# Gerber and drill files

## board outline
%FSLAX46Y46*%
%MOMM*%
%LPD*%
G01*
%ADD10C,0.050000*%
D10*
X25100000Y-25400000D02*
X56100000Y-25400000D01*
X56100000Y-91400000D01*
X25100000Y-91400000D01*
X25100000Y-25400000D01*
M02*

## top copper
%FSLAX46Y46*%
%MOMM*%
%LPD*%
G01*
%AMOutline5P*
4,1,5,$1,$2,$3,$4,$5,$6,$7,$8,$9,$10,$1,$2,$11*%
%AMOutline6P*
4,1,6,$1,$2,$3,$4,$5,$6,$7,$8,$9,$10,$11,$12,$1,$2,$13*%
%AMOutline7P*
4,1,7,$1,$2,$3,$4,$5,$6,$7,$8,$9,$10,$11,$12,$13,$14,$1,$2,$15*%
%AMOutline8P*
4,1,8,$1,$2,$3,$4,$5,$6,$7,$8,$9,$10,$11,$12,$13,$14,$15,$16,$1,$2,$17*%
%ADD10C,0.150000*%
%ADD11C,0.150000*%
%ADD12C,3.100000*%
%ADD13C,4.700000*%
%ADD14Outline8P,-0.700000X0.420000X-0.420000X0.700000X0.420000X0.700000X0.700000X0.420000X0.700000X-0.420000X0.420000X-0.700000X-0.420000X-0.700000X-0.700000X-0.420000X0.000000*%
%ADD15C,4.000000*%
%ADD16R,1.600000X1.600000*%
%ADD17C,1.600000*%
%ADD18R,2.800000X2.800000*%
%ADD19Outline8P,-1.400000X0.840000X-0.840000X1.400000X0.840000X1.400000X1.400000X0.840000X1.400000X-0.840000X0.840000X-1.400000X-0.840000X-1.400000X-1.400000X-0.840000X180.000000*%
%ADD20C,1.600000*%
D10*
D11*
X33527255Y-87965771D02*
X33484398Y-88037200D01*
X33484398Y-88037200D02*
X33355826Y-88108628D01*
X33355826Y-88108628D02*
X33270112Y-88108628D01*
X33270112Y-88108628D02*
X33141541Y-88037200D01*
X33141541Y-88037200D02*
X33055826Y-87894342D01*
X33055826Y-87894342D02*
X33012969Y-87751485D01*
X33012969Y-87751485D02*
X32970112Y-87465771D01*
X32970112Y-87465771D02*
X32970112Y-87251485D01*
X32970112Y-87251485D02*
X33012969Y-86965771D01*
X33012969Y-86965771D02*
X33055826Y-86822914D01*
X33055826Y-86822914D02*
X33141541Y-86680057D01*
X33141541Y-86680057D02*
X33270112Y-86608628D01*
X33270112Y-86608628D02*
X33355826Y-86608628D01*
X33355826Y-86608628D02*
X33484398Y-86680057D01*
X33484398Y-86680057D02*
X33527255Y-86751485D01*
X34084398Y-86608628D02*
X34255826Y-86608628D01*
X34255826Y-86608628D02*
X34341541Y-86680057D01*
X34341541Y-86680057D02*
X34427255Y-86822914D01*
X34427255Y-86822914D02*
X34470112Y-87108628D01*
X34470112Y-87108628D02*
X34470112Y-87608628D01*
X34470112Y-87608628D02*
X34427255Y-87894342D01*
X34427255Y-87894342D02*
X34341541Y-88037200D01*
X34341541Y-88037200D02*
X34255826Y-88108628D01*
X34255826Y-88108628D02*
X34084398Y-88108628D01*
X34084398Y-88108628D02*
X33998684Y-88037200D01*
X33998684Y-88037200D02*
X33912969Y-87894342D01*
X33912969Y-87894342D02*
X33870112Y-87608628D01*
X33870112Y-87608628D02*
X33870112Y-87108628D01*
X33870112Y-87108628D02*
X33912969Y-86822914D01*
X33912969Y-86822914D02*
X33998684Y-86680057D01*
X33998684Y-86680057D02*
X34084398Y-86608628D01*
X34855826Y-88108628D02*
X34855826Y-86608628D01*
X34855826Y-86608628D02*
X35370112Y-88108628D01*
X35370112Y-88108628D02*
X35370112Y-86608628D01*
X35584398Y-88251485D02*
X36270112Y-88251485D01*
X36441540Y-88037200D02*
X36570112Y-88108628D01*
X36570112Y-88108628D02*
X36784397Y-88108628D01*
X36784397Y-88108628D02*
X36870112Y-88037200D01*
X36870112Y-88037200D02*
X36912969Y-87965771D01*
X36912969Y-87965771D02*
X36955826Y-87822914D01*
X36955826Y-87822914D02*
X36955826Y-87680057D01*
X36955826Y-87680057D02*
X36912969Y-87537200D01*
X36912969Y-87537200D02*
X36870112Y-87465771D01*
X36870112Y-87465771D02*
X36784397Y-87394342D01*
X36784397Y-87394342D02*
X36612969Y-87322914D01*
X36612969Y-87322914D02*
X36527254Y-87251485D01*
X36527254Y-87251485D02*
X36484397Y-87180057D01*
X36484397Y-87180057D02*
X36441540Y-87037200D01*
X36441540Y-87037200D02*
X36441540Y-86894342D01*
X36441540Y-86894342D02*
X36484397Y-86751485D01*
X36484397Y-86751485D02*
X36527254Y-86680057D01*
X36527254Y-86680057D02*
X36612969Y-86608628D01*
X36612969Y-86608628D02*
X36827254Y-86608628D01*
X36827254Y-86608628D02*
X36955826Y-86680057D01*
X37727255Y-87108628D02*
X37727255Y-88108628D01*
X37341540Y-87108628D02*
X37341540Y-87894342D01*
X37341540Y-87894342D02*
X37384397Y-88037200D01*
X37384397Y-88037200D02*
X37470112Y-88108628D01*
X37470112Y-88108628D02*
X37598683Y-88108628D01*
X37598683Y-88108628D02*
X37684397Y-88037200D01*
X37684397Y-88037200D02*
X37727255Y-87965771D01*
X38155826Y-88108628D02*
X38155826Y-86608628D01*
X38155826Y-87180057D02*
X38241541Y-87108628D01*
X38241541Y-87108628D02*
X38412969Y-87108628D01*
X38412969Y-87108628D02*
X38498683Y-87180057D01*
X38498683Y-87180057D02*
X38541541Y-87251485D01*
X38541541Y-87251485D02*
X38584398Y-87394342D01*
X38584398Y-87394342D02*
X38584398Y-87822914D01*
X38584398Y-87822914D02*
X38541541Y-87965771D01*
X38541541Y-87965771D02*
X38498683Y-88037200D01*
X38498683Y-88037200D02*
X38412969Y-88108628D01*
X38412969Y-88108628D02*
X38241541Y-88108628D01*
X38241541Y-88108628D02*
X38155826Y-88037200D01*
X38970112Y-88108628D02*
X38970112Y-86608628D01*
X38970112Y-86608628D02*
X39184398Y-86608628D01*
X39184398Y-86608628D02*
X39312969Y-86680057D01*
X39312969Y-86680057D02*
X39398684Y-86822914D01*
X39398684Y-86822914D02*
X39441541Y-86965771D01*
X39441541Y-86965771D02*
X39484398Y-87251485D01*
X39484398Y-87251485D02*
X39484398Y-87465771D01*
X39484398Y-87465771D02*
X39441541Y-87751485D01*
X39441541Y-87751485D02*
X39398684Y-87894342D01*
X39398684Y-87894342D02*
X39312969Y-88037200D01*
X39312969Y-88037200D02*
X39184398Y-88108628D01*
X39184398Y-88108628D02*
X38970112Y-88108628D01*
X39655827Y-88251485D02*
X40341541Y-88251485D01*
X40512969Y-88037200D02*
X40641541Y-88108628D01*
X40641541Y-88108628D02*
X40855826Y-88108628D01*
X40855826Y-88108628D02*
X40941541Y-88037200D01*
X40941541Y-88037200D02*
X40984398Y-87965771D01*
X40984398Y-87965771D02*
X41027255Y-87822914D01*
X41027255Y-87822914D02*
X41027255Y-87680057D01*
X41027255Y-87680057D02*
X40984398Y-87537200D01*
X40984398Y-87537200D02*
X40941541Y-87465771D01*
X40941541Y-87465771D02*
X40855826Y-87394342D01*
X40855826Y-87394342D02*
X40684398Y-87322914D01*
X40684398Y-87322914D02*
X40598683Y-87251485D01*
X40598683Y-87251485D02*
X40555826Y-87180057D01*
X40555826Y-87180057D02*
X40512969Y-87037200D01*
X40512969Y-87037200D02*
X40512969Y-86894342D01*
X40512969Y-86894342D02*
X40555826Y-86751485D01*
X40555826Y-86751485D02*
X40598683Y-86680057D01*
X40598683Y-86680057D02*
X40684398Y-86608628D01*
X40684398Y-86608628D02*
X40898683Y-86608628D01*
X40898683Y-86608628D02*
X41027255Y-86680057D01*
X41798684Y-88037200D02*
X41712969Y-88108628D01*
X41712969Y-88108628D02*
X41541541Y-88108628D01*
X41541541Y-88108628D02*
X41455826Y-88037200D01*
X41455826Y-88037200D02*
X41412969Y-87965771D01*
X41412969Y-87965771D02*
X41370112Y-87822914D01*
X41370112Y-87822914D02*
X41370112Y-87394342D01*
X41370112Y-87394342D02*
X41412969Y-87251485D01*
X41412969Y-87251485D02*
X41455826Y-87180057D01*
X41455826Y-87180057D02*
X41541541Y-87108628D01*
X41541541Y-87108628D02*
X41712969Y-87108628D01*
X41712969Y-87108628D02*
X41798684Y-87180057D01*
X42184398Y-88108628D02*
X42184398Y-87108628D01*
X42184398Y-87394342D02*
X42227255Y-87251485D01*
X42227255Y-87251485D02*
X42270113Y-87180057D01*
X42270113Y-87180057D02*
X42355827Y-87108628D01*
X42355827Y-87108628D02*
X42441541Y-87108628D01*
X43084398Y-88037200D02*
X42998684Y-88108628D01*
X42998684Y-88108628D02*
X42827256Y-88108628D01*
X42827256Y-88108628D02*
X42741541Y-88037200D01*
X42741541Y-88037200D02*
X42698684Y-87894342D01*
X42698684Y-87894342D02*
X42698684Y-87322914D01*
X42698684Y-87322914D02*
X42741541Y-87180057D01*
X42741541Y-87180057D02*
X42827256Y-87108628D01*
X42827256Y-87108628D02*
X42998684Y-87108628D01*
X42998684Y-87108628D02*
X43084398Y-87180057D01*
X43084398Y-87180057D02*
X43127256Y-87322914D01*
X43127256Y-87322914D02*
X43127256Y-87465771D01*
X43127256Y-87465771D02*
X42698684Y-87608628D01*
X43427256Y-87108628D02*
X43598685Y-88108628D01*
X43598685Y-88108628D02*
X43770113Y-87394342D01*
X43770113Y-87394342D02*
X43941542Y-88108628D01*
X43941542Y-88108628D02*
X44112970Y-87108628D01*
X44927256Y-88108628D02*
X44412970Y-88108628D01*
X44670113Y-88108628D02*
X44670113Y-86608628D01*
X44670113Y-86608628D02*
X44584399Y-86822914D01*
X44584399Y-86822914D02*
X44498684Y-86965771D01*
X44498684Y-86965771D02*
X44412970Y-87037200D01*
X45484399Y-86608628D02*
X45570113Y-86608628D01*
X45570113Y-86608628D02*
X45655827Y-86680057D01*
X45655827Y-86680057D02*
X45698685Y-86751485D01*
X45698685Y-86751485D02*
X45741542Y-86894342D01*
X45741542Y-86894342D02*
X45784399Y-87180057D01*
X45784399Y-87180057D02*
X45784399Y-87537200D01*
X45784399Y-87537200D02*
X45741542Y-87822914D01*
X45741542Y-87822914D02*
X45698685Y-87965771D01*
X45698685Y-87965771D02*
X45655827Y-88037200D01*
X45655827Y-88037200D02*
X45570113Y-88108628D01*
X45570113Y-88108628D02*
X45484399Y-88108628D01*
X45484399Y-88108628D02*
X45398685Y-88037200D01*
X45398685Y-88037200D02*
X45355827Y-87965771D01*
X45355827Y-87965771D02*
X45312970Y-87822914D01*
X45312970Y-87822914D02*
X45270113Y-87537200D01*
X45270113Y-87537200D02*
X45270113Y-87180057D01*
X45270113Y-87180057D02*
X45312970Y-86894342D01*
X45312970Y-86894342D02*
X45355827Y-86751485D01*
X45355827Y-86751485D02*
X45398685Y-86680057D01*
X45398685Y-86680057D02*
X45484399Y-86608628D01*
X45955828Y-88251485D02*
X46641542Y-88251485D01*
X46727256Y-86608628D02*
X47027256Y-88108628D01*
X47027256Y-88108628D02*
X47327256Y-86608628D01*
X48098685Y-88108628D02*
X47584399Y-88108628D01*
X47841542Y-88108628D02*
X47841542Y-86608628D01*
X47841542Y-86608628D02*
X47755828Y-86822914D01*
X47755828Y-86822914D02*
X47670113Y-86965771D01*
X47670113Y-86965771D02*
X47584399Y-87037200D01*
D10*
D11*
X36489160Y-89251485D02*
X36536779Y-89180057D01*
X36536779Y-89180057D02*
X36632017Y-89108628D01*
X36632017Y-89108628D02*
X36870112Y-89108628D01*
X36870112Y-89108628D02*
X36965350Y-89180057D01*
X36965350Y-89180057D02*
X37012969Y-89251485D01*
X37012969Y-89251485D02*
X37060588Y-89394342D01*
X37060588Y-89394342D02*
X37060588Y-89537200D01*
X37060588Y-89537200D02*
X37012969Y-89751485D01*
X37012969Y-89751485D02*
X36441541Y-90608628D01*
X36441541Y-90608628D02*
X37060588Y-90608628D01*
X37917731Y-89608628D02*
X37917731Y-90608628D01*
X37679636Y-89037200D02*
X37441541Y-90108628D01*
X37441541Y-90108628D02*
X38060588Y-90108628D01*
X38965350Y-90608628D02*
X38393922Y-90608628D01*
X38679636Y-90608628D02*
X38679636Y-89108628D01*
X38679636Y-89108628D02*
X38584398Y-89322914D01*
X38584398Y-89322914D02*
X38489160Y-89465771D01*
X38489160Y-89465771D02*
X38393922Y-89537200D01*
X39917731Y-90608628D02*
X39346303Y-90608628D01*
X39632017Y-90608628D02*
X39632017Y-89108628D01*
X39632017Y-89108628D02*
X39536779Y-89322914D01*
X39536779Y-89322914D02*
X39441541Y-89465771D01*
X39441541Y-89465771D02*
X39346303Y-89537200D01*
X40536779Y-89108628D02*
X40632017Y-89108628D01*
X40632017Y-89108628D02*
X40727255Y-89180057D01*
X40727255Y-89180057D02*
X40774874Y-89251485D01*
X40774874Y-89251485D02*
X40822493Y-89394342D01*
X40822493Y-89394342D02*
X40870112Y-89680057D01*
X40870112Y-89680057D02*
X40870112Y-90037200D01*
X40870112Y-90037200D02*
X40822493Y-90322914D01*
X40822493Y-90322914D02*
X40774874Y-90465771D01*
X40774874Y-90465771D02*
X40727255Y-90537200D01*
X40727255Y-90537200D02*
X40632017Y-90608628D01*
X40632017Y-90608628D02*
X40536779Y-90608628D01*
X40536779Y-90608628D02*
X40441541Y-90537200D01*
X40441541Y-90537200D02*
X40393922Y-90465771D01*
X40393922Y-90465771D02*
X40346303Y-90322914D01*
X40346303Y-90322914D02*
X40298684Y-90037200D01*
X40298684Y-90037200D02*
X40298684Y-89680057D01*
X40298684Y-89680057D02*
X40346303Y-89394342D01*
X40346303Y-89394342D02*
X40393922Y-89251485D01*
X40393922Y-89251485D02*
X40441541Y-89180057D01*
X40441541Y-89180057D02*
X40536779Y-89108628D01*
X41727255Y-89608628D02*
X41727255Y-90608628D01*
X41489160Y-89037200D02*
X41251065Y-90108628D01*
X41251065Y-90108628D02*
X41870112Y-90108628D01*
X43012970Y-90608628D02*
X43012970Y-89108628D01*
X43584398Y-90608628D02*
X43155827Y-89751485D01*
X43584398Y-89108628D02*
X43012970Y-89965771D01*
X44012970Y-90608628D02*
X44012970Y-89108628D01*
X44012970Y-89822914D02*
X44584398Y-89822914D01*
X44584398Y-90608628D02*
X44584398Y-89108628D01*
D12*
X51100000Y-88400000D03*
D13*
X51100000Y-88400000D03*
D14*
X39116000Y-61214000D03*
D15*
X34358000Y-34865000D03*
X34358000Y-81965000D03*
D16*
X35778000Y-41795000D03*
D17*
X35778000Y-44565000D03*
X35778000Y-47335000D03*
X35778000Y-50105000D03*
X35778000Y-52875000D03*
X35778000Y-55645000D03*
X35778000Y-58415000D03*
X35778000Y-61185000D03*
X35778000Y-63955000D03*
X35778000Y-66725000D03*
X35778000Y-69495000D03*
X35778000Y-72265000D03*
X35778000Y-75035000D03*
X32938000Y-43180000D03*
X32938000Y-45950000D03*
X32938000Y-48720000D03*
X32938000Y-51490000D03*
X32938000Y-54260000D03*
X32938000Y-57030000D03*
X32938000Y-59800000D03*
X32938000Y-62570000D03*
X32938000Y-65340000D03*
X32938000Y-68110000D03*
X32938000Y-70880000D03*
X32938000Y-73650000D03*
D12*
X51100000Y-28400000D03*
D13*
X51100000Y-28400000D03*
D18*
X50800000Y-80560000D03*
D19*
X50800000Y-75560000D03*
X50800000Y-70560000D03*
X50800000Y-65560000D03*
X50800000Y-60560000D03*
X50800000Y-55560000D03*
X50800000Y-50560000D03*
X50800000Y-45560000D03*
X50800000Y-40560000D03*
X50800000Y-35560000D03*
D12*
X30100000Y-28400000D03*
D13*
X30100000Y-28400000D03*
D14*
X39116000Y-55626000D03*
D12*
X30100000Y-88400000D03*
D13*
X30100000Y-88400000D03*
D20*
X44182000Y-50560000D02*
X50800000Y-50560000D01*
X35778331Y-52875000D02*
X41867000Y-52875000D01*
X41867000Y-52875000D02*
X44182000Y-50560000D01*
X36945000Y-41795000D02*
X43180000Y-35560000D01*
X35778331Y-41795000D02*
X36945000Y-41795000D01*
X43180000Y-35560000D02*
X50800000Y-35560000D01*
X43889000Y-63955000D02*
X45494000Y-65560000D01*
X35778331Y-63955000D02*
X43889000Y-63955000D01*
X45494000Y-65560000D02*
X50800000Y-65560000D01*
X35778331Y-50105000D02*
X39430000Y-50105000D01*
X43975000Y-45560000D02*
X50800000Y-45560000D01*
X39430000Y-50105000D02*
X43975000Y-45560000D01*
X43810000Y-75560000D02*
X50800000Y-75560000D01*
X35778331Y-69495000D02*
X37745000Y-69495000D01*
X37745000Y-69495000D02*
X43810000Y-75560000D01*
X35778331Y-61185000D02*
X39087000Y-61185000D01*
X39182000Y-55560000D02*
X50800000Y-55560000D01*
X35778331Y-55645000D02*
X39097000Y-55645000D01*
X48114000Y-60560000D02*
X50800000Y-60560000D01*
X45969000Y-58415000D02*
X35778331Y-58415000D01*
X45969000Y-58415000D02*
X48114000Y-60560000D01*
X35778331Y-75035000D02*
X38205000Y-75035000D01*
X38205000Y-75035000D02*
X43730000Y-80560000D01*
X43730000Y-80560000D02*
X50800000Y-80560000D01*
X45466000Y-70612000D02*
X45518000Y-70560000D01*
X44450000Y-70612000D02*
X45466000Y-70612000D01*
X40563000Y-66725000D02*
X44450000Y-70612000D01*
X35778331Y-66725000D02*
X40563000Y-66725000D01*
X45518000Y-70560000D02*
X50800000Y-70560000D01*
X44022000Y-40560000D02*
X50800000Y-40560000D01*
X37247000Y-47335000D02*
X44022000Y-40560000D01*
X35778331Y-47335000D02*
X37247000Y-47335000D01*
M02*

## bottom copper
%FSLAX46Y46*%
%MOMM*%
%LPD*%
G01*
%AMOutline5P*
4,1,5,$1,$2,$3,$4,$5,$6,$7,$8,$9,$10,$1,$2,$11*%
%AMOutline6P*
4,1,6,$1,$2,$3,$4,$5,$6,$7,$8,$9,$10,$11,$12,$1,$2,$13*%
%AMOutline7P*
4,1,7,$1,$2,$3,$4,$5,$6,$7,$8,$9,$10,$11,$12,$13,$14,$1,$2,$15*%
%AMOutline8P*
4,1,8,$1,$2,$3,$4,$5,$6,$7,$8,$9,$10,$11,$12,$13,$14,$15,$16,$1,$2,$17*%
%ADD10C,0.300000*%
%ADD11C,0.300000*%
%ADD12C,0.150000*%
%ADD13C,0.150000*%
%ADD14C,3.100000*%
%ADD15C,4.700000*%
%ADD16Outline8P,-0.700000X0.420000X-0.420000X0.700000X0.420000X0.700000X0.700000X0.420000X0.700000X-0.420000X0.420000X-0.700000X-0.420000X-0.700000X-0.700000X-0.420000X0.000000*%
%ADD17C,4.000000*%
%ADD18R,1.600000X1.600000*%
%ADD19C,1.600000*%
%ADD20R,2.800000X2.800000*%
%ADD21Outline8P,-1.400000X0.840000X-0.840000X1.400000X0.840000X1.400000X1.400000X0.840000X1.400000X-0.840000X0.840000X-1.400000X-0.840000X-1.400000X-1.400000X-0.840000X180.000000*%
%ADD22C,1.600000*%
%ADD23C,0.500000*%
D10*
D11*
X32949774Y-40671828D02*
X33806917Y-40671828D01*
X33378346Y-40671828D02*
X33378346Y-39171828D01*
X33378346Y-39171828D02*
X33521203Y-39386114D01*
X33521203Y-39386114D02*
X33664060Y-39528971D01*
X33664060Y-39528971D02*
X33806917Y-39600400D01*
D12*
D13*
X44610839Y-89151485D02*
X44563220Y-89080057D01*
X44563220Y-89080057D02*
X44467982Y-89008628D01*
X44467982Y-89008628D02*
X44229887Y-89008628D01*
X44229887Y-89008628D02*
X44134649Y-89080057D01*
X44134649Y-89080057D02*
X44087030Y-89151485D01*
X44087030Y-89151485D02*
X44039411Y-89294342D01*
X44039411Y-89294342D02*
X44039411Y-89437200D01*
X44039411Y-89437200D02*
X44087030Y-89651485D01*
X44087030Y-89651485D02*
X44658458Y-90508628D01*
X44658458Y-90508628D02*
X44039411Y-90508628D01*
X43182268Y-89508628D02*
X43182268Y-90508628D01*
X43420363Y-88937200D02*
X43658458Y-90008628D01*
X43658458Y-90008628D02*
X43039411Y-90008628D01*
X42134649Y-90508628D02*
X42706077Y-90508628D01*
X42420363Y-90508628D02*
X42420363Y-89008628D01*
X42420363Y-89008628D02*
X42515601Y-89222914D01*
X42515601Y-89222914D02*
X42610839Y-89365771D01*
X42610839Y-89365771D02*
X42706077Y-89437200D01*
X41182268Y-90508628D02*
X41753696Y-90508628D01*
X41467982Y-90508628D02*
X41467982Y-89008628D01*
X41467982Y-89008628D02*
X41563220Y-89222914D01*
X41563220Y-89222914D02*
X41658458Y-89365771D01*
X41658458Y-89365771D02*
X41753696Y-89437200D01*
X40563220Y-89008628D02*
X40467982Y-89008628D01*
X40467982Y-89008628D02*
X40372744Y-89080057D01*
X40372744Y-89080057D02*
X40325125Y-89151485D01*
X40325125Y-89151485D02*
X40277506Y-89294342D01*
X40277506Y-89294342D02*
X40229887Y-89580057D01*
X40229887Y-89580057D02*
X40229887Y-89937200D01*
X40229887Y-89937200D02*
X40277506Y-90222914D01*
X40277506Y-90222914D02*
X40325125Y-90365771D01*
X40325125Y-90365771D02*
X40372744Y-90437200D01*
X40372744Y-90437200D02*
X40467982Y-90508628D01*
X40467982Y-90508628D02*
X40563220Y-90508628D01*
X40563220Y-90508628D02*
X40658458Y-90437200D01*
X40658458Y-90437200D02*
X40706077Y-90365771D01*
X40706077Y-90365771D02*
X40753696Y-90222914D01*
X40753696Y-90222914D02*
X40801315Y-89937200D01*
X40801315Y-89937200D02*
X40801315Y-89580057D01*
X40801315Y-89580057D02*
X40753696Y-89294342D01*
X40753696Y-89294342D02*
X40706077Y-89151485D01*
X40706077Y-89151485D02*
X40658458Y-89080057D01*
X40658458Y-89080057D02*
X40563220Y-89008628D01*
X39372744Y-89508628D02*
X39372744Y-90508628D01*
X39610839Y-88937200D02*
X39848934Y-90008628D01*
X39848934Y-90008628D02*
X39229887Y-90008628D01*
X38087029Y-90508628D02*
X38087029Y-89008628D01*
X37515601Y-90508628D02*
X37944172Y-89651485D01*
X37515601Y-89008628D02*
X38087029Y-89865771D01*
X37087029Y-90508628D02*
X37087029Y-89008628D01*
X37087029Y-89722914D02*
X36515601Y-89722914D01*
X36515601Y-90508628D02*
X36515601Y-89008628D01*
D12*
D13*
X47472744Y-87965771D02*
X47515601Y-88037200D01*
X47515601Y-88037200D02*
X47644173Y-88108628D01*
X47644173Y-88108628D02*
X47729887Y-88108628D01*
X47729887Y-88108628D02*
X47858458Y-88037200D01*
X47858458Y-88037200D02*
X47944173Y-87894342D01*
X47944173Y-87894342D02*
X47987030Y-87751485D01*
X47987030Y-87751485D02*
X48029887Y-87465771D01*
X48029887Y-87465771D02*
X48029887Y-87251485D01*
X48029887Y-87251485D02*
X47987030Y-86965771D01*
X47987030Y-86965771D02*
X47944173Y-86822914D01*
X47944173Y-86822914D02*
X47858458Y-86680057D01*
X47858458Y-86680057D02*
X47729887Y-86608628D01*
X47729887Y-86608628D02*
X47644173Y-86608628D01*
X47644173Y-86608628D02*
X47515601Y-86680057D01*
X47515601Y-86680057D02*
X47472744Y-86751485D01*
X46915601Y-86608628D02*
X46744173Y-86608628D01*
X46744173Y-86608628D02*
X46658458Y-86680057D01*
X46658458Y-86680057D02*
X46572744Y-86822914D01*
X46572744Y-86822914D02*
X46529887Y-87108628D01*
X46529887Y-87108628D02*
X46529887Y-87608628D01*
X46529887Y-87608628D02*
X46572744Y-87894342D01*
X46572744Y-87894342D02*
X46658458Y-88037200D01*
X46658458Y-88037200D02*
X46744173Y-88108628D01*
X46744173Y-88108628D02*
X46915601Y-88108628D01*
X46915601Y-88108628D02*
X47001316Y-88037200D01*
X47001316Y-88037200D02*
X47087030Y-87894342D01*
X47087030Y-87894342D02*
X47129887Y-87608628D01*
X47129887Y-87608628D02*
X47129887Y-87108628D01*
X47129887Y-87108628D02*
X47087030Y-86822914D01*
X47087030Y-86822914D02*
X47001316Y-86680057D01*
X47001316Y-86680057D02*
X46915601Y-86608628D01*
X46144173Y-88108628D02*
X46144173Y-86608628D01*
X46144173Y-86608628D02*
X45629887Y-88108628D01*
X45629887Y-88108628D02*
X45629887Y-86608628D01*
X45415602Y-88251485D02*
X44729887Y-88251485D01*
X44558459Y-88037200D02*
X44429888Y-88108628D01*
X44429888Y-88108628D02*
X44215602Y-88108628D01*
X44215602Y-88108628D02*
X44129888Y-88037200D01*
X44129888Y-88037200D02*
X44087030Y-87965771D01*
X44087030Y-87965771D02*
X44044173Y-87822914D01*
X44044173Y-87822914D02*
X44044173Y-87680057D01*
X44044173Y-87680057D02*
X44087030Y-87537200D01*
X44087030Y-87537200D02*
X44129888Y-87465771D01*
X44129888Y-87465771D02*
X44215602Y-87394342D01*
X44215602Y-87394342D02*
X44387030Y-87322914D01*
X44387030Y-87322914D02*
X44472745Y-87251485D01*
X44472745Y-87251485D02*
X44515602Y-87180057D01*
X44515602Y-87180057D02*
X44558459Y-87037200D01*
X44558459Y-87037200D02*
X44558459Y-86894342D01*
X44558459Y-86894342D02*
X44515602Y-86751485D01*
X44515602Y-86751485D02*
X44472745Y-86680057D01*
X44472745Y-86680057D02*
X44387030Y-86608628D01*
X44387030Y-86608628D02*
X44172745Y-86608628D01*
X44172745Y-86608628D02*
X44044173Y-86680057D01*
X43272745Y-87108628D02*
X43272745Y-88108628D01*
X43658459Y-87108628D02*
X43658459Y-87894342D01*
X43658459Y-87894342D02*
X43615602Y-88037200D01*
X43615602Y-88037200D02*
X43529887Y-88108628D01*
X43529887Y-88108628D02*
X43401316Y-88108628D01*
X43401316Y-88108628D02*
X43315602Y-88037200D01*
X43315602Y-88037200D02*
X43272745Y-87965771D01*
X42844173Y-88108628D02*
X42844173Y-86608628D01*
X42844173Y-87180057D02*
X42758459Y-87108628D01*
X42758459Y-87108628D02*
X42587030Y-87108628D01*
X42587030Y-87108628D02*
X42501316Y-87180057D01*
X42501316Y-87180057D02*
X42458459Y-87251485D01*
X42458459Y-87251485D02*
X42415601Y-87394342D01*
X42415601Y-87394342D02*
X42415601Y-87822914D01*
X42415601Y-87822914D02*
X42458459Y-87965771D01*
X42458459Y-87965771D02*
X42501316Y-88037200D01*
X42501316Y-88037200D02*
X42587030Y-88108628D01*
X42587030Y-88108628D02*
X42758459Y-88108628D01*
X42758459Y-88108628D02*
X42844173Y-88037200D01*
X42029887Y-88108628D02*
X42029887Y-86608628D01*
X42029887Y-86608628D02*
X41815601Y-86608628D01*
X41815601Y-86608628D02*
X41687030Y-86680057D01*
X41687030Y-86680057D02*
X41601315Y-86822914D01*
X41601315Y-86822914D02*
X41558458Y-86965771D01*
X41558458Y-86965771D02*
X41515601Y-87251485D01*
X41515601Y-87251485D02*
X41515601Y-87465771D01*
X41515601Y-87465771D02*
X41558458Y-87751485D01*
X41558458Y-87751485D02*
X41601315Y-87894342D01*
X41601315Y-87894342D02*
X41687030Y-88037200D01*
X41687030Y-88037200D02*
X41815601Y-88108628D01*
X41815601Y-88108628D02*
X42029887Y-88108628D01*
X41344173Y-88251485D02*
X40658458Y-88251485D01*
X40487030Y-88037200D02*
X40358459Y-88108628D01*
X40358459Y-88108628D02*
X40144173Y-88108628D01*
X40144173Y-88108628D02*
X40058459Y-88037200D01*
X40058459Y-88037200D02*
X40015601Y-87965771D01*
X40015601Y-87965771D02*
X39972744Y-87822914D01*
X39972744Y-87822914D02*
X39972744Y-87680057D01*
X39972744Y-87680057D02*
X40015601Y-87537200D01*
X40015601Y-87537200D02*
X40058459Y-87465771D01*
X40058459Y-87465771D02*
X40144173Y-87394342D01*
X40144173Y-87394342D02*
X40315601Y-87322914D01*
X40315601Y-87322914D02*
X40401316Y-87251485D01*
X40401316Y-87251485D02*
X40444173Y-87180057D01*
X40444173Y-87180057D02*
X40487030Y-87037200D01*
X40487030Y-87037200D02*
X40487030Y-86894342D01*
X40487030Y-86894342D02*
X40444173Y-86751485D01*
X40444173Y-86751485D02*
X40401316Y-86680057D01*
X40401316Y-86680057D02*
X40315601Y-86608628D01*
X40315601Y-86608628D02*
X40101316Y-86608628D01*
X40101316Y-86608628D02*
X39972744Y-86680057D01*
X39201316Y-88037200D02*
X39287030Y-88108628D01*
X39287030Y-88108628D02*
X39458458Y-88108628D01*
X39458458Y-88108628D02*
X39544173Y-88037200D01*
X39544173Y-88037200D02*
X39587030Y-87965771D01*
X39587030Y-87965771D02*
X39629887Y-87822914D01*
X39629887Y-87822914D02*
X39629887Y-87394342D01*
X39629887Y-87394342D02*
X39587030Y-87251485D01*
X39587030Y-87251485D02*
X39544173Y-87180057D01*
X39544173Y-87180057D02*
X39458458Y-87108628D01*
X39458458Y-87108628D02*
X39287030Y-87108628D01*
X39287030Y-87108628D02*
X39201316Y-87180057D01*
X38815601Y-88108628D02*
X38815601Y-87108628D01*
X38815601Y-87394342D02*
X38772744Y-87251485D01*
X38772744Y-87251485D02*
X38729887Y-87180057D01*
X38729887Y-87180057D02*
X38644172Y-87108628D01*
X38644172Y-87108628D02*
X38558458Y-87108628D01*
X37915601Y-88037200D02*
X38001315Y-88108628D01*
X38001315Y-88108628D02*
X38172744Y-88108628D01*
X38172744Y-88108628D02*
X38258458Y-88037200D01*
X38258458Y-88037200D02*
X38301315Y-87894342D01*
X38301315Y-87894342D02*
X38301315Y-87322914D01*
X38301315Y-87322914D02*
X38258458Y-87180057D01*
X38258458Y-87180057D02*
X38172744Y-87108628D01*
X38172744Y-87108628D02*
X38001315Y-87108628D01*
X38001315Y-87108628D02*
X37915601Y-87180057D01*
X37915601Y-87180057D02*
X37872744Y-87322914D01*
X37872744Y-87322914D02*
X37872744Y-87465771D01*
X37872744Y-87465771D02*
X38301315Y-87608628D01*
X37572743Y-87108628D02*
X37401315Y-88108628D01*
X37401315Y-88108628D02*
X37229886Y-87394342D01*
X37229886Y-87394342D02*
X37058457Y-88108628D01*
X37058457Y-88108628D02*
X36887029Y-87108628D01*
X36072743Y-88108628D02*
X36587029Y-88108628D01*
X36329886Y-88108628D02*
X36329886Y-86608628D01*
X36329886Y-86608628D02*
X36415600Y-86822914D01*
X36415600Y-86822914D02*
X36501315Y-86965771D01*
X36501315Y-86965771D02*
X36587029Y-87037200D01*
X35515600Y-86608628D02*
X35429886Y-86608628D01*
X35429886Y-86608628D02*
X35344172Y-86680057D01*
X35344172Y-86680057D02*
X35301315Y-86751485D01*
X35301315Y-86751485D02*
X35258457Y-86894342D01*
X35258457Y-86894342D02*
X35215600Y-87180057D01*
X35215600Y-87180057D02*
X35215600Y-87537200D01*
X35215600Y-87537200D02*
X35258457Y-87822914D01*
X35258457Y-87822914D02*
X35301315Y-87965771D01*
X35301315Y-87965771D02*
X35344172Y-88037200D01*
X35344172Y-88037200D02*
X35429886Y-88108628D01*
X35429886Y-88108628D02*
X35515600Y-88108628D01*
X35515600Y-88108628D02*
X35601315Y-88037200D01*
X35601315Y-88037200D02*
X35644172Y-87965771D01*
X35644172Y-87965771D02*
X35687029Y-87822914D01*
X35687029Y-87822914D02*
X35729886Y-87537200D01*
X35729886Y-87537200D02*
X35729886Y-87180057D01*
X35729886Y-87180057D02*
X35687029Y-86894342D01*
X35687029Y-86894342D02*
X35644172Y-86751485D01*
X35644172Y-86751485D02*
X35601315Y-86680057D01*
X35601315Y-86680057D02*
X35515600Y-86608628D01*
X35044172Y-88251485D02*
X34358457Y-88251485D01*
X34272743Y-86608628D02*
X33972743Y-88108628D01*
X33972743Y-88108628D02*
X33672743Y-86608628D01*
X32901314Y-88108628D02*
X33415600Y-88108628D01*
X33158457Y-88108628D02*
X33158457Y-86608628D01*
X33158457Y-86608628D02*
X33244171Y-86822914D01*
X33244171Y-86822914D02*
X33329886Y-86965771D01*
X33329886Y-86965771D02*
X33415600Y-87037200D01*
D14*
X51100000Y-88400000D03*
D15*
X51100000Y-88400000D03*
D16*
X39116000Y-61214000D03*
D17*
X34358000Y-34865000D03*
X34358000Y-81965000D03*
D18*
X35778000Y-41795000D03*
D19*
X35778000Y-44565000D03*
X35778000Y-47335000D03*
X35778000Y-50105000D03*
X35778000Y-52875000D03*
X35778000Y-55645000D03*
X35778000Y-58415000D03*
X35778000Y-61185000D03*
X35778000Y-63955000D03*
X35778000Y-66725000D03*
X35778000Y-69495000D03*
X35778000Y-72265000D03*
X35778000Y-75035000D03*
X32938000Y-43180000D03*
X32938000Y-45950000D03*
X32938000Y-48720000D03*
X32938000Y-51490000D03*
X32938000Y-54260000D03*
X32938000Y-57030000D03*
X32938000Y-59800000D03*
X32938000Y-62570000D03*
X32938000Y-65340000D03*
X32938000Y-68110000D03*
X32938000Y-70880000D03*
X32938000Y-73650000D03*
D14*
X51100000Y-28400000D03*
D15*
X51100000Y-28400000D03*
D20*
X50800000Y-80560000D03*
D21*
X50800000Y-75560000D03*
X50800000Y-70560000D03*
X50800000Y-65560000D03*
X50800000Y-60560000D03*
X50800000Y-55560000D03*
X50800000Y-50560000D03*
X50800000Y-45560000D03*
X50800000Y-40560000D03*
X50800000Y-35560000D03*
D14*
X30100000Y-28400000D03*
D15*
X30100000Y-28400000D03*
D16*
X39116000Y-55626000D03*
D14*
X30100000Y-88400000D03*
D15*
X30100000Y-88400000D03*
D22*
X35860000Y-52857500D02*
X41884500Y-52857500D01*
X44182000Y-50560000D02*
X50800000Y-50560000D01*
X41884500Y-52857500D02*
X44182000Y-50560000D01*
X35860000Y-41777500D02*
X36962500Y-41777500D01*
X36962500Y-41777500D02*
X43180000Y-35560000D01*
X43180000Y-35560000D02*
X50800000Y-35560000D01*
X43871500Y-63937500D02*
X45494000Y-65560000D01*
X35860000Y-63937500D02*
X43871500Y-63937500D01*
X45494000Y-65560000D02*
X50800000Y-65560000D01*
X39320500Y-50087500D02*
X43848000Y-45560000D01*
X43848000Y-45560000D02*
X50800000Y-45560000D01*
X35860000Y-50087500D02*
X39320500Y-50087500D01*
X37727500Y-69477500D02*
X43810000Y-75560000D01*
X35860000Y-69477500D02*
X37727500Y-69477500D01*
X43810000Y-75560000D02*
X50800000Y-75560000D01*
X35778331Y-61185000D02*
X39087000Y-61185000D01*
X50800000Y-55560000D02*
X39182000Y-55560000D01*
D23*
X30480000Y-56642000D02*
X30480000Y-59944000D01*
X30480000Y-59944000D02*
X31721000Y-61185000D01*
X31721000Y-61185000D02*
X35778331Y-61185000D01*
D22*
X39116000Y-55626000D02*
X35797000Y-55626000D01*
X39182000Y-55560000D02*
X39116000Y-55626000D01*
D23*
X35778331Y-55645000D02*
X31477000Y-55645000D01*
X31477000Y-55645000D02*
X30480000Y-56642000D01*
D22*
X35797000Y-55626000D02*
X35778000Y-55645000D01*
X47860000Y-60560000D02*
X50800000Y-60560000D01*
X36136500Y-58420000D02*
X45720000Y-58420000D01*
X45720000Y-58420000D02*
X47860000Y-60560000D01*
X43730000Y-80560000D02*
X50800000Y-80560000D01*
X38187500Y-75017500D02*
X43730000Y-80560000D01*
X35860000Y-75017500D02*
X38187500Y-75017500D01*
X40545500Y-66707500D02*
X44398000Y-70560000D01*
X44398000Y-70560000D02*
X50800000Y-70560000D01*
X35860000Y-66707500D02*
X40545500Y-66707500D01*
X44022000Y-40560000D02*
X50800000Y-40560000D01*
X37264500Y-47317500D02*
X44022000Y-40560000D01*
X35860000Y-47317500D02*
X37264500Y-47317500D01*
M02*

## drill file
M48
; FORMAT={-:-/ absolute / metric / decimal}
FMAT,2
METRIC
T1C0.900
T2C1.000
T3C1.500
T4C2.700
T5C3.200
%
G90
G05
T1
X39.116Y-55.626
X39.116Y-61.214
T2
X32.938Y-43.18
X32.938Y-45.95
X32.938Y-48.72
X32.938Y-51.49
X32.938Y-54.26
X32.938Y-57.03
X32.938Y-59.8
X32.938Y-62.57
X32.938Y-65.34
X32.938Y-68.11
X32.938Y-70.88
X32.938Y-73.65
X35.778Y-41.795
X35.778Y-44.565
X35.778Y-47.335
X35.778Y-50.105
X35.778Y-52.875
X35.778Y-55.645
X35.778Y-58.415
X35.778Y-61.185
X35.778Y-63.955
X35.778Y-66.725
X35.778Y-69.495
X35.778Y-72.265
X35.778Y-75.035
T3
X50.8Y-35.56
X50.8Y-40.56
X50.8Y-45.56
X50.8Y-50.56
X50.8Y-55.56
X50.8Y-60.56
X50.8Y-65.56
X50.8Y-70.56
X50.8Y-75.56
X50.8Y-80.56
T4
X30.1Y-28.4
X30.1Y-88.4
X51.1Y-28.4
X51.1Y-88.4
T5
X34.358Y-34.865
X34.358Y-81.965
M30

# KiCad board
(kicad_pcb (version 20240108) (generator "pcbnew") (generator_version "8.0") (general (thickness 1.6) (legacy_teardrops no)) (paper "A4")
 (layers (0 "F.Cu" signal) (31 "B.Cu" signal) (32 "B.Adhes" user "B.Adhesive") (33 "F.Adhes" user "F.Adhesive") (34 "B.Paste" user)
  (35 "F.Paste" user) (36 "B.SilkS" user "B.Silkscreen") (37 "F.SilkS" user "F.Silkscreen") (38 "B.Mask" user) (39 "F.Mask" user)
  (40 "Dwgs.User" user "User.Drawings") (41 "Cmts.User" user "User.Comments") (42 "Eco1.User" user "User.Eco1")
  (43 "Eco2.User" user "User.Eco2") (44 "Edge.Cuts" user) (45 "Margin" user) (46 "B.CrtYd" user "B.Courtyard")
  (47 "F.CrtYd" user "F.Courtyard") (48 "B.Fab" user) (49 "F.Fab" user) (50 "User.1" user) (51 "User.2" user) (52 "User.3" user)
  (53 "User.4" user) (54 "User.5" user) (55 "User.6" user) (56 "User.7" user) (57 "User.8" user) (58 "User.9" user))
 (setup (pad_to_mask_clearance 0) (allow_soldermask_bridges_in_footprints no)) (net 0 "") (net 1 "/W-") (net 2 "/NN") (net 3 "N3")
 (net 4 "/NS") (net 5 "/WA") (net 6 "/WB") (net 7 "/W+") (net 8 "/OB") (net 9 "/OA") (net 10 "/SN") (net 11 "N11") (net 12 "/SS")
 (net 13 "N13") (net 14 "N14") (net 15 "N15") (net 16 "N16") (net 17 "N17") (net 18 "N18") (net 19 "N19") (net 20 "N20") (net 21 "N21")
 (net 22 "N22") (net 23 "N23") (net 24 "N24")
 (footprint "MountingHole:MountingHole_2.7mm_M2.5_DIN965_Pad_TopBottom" (layer "F.Cu") (at 51.1 88.4)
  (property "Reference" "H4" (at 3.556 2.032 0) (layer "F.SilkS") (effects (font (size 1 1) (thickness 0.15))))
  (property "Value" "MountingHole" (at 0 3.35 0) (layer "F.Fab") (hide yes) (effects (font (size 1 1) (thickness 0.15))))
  (pad "1" thru_hole circle (at 0 0) (size 3.1 3.1) (drill 2.7) (layers "*.Cu" "*.Mask") (remove_unused_layers no))
  (pad "1" connect circle (at 0 0) (size 4.7 4.7) (layers "F.Cu" "F.Mask"))
  (pad "1" connect circle (at 0 0) (size 4.7 4.7) (layers "B.Cu" "B.Mask")))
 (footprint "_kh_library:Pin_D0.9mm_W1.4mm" (layer "F.Cu") (at 39.116 61.214)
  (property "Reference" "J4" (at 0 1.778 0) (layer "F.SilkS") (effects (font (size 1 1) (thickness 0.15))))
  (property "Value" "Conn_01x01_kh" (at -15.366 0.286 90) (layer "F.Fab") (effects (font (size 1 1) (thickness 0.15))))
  (pad "1" thru_hole roundrect (at 0 0) (size 1.4 1.4) (drill 0.9) (layers "*.Cu" "*.Mask") (remove_unused_layers no) (roundrect_rratio 0)
   (chamfer_ratio 0.2) (chamfer top_left top_right bottom_left bottom_right) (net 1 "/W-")))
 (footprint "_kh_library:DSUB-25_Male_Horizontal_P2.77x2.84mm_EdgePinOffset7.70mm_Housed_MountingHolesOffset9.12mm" (layer "F.Cu")
  (at 35.778 41.795 -90)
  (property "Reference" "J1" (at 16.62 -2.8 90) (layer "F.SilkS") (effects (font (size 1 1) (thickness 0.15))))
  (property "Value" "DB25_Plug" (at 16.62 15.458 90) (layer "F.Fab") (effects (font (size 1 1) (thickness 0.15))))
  (pad "0" thru_hole circle (at -6.93 1.42 270) (size 4 4) (drill 3.2) (layers "*.Cu" "*.Mask") (remove_unused_layers no))
  (pad "0" thru_hole circle (at 40.17 1.42 270) (size 4 4) (drill 3.2) (layers "*.Cu" "*.Mask") (remove_unused_layers no))
  (pad "1" thru_hole rect (at 0 0 270) (size 1.6 1.6) (drill 1) (layers "*.Cu" "*.Mask") (remove_unused_layers no) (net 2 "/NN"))
  (pad "2" thru_hole circle (at 2.77 0 270) (size 1.6 1.6) (drill 1) (layers "*.Cu" "*.Mask") (remove_unused_layers no) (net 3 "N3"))
  (pad "3" thru_hole circle (at 5.54 0 270) (size 1.6 1.6) (drill 1) (layers "*.Cu" "*.Mask") (remove_unused_layers no) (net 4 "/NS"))
  (pad "4" thru_hole circle (at 8.31 0 270) (size 1.6 1.6) (drill 1) (layers "*.Cu" "*.Mask") (remove_unused_layers no) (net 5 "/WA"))
  (pad "5" thru_hole circle (at 11.08 0 270) (size 1.6 1.6) (drill 1) (layers "*.Cu" "*.Mask") (remove_unused_layers no) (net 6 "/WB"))
  (pad "6" thru_hole circle (at 13.85 0 270) (size 1.6 1.6) (drill 1) (layers "*.Cu" "*.Mask") (remove_unused_layers no) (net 1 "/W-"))
  (pad "7" thru_hole circle (at 16.62 0 270) (size 1.6 1.6) (drill 1) (layers "*.Cu" "*.Mask") (remove_unused_layers no) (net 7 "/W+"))
  (pad "8" thru_hole circle (at 19.39 0 270) (size 1.6 1.6) (drill 1) (layers "*.Cu" "*.Mask") (remove_unused_layers no) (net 1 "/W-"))
  (pad "9" thru_hole circle (at 22.16 0 270) (size 1.6 1.6) (drill 1) (layers "*.Cu" "*.Mask") (remove_unused_layers no) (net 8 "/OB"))
  (pad "10" thru_hole circle (at 24.93 0 270) (size 1.6 1.6) (drill 1) (layers "*.Cu" "*.Mask") (remove_unused_layers no) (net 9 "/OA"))
  (pad "11" thru_hole circle (at 27.7 0 270) (size 1.6 1.6) (drill 1) (layers "*.Cu" "*.Mask") (remove_unused_layers no) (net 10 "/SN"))
  (pad "12" thru_hole circle (at 30.47 0 270) (size 1.6 1.6) (drill 1) (layers "*.Cu" "*.Mask") (remove_unused_layers no) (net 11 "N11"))
  (pad "13" thru_hole circle (at 33.24 0 270) (size 1.6 1.6) (drill 1) (layers "*.Cu" "*.Mask") (remove_unused_layers no) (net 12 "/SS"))
  (pad "14" thru_hole circle (at 1.385 2.84 270) (size 1.6 1.6) (drill 1) (layers "*.Cu" "*.Mask") (remove_unused_layers no) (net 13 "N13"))
  (pad "15" thru_hole circle (at 4.155 2.84 270) (size 1.6 1.6) (drill 1) (layers "*.Cu" "*.Mask") (remove_unused_layers no) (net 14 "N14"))
  (pad "16" thru_hole circle (at 6.925 2.84 270) (size 1.6 1.6) (drill 1) (layers "*.Cu" "*.Mask") (remove_unused_layers no) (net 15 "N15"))
  (pad "17" thru_hole circle (at 9.695 2.84 270) (size 1.6 1.6) (drill 1) (layers "*.Cu" "*.Mask") (remove_unused_layers no) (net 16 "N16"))
  (pad "18" thru_hole circle (at 12.465 2.84 270) (size 1.6 1.6) (drill 1) (layers "*.Cu" "*.Mask") (remove_unused_layers no) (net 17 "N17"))
  (pad "19" thru_hole circle (at 15.235 2.84 270) (size 1.6 1.6) (drill 1) (layers "*.Cu" "*.Mask") (remove_unused_layers no) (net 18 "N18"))
  (pad "20" thru_hole circle (at 18.005 2.84 270) (size 1.6 1.6) (drill 1) (layers "*.Cu" "*.Mask") (remove_unused_layers no) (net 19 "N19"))
  (pad "21" thru_hole circle (at 20.775 2.84 270) (size 1.6 1.6) (drill 1) (layers "*.Cu" "*.Mask") (remove_unused_layers no) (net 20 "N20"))
  (pad "22" thru_hole circle (at 23.545 2.84 270) (size 1.6 1.6) (drill 1) (layers "*.Cu" "*.Mask") (remove_unused_layers no) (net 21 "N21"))
  (pad "23" thru_hole circle (at 26.315 2.84 270) (size 1.6 1.6) (drill 1) (layers "*.Cu" "*.Mask") (remove_unused_layers no) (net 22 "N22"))
  (pad "24" thru_hole circle (at 29.085 2.84 270) (size 1.6 1.6) (drill 1) (layers "*.Cu" "*.Mask") (remove_unused_layers no) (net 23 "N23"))
  (pad "25" thru_hole circle (at 31.855 2.84 270) (size 1.6 1.6) (drill 1) (layers "*.Cu" "*.Mask") (remove_unused_layers no) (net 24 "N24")))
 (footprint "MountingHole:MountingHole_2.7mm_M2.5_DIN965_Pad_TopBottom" (layer "F.Cu") (at 51.1 28.4)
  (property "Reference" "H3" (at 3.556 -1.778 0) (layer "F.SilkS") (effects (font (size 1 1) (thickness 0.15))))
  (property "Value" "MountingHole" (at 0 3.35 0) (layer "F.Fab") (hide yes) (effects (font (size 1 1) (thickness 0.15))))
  (pad "1" thru_hole circle (at 0 0) (size 3.1 3.1) (drill 2.7) (layers "*.Cu" "*.Mask") (remove_unused_layers no))
  (pad "1" connect circle (at 0 0) (size 4.7 4.7) (layers "F.Cu" "F.Mask"))
  (pad "1" connect circle (at 0 0) (size 4.7 4.7) (layers "B.Cu" "B.Mask")))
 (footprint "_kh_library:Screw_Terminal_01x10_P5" (layer "F.Cu") (at 50.8 80.56 180)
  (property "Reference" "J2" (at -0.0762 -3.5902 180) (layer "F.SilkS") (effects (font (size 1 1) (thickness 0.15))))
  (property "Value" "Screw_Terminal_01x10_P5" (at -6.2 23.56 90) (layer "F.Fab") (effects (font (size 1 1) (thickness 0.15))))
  (pad "1" thru_hole rect (at 0 0 180) (size 2.8 2.8) (drill 1.5) (layers "*.Cu" "*.Mask") (remove_unused_layers no) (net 12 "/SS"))
  (pad "2" thru_hole roundrect (at 0 5 180) (size 2.8 2.8) (drill 1.5) (layers "*.Cu" "*.Mask") (remove_unused_layers no)
   (roundrect_rratio 0) (chamfer_ratio 0.2) (chamfer top_left top_right bottom_left bottom_right) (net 10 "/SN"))
  (pad "3" thru_hole roundrect (at 0 10 180) (size 2.8 2.8) (drill 1.5) (layers "*.Cu" "*.Mask") (remove_unused_layers no)
   (roundrect_rratio 0) (chamfer_ratio 0.2) (chamfer top_left top_right bottom_left bottom_right) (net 9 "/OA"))
  (pad "4" thru_hole roundrect (at 0 15 180) (size 2.8 2.8) (drill 1.5) (layers "*.Cu" "*.Mask") (remove_unused_layers no)
   (roundrect_rratio 0) (chamfer_ratio 0.2) (chamfer top_left top_right bottom_left bottom_right) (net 8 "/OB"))
  (pad "5" thru_hole roundrect (at 0 20 180) (size 2.8 2.8) (drill 1.5) (layers "*.Cu" "*.Mask") (remove_unused_layers no)
   (roundrect_rratio 0) (chamfer_ratio 0.2) (chamfer top_left top_right bottom_left bottom_right) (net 7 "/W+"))
  (pad "6" thru_hole roundrect (at 0 25 180) (size 2.8 2.8) (drill 1.5) (layers "*.Cu" "*.Mask") (remove_unused_layers no)
   (roundrect_rratio 0) (chamfer_ratio 0.2) (chamfer top_left top_right bottom_left bottom_right) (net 1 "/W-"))
  (pad "7" thru_hole roundrect (at 0 30 180) (size 2.8 2.8) (drill 1.5) (layers "*.Cu" "*.Mask") (remove_unused_layers no)
   (roundrect_rratio 0) (chamfer_ratio 0.2) (chamfer top_left top_right bottom_left bottom_right) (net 6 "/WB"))
  (pad "8" thru_hole roundrect (at 0 35 180) (size 2.8 2.8) (drill 1.5) (layers "*.Cu" "*.Mask") (remove_unused_layers no)
   (roundrect_rratio 0) (chamfer_ratio 0.2) (chamfer top_left top_right bottom_left bottom_right) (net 5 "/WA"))
  (pad "9" thru_hole roundrect (at 0 40 180) (size 2.8 2.8) (drill 1.5) (layers "*.Cu" "*.Mask") (remove_unused_layers no)
   (roundrect_rratio 0) (chamfer_ratio 0.2) (chamfer top_left top_right bottom_left bottom_right) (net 4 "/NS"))
  (pad "10" thru_hole roundrect (at 0 45 180) (size 2.8 2.8) (drill 1.5) (layers "*.Cu" "*.Mask") (remove_unused_layers no)
   (roundrect_rratio 0) (chamfer_ratio 0.2) (chamfer top_left top_right bottom_left bottom_right) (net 2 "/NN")))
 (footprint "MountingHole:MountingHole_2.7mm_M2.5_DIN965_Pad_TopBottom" (layer "F.Cu") (at 30.1 28.4)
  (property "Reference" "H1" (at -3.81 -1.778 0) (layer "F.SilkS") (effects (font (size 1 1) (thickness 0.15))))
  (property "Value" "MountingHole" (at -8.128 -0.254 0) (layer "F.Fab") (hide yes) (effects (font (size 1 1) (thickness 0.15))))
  (pad "1" thru_hole circle (at 0 0) (size 3.1 3.1) (drill 2.7) (layers "*.Cu" "*.Mask") (remove_unused_layers no))
  (pad "1" connect circle (at 0 0) (size 4.7 4.7) (layers "F.Cu" "F.Mask"))
  (pad "1" connect circle (at 0 0) (size 4.7 4.7) (layers "B.Cu" "B.Mask")))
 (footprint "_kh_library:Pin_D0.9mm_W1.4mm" (layer "F.Cu") (at 39.116 55.626)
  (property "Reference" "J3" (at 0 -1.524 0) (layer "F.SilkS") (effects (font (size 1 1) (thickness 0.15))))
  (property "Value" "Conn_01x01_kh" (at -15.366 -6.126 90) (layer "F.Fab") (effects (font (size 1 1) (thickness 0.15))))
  (pad "1" thru_hole roundrect (at 0 0) (size 1.4 1.4) (drill 0.9) (layers "*.Cu" "*.Mask") (remove_unused_layers no) (roundrect_rratio 0)
   (chamfer_ratio 0.2) (chamfer top_left top_right bottom_left bottom_right) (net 1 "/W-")))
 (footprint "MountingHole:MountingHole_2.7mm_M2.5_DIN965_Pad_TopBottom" (layer "F.Cu") (at 30.1 88.4)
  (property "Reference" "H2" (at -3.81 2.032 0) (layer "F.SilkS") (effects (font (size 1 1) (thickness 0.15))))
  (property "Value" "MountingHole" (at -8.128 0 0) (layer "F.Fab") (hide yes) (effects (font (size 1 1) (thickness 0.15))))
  (pad "1" thru_hole circle (at 0 0) (size 3.1 3.1) (drill 2.7) (layers "*.Cu" "*.Mask") (remove_unused_layers no))
  (pad "1" connect circle (at 0 0) (size 4.7 4.7) (layers "F.Cu" "F.Mask"))
  (pad "1" connect circle (at 0 0) (size 4.7 4.7) (layers "B.Cu" "B.Mask")))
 (gr_rect (start 25.1 25.4) (end 56.1 91.4) (stroke (width 0.05) (type default)) (fill none) (layer "Edge.Cuts"))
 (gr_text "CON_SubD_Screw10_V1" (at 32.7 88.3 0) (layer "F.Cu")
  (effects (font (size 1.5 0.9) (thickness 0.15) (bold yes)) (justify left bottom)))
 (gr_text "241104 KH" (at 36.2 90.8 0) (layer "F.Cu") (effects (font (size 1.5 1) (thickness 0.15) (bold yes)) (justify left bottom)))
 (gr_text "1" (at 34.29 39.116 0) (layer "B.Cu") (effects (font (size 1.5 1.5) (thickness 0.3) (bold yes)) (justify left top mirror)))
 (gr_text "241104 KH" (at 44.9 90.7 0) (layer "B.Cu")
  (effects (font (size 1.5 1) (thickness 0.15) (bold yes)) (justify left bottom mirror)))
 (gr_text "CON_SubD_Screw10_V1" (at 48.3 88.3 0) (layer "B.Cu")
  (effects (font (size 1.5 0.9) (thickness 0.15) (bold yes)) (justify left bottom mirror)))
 (segment (start 44.182 50.56) (end 50.8 50.56) (width 1.6) (layer "F.Cu") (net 6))
 (segment (start 35.778331 52.875) (end 41.867 52.875) (width 1.6) (layer "F.Cu") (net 6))
 (segment (start 41.867 52.875) (end 44.182 50.56) (width 1.6) (layer "F.Cu") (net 6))
 (segment (start 35.86 52.8575) (end 41.8845 52.8575) (width 1.6) (layer "B.Cu") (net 6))
 (segment (start 44.182 50.56) (end 50.8 50.56) (width 1.6) (layer "B.Cu") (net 6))
 (segment (start 41.8845 52.8575) (end 44.182 50.56) (width 1.6) (layer "B.Cu") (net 6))
 (segment (start 36.945 41.795) (end 43.18 35.56) (width 1.6) (layer "F.Cu") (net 2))
 (segment (start 35.778331 41.795) (end 36.945 41.795) (width 1.6) (layer "F.Cu") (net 2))
 (segment (start 43.18 35.56) (end 50.8 35.56) (width 1.6) (layer "F.Cu") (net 2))
 (segment (start 35.86 41.7775) (end 36.9625 41.7775) (width 1.6) (layer "B.Cu") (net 2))
 (segment (start 36.9625 41.7775) (end 43.18 35.56) (width 1.6) (layer "B.Cu") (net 2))
 (segment (start 43.18 35.56) (end 50.8 35.56) (width 1.6) (layer "B.Cu") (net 2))
 (segment (start 43.889 63.955) (end 45.494 65.56) (width 1.6) (layer "F.Cu") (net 8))
 (segment (start 35.778331 63.955) (end 43.889 63.955) (width 1.6) (layer "F.Cu") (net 8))
 (segment (start 45.494 65.56) (end 50.8 65.56) (width 1.6) (layer "F.Cu") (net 8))
 (segment (start 43.8715 63.9375) (end 45.494 65.56) (width 1.6) (layer "B.Cu") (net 8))
 (segment (start 35.86 63.9375) (end 43.8715 63.9375) (width 1.6) (layer "B.Cu") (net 8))
 (segment (start 45.494 65.56) (end 50.8 65.56) (width 1.6) (layer "B.Cu") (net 8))
 (segment (start 35.778331 50.105) (end 39.43 50.105) (width 1.6) (layer "F.Cu") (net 5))
 (segment (start 43.975 45.56) (end 50.8 45.56) (width 1.6) (layer "F.Cu") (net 5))
 (segment (start 39.43 50.105) (end 43.975 45.56) (width 1.6) (layer "F.Cu") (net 5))
 (segment (start 39.3205 50.0875) (end 43.848 45.56) (width 1.6) (layer "B.Cu") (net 5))
 (segment (start 43.848 45.56) (end 50.8 45.56) (width 1.6) (layer "B.Cu") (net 5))
 (segment (start 35.86 50.0875) (end 39.3205 50.0875) (width 1.6) (layer "B.Cu") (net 5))
 (segment (start 43.81 75.56) (end 50.8 75.56) (width 1.6) (layer "F.Cu") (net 10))
 (segment (start 35.778331 69.495) (end 37.745 69.495) (width 1.6) (layer "F.Cu") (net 10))
 (segment (start 37.745 69.495) (end 43.81 75.56) (width 1.6) (layer "F.Cu") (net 10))
 (segment (start 37.7275 69.4775) (end 43.81 75.56) (width 1.6) (layer "B.Cu") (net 10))
 (segment (start 35.86 69.4775) (end 37.7275 69.4775) (width 1.6) (layer "B.Cu") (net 10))
 (segment (start 43.81 75.56) (end 50.8 75.56) (width 1.6) (layer "B.Cu") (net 10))
 (segment (start 35.778331 61.185) (end 39.087 61.185) (width 1.6) (layer "F.Cu") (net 1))
 (segment (start 39.182 55.56) (end 50.8 55.56) (width 1.6) (layer "F.Cu") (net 1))
 (segment (start 35.778331 55.645) (end 39.097 55.645) (width 1.6) (layer "F.Cu") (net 1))
 (segment (start 35.778331 61.185) (end 39.087 61.185) (width 1.6) (layer "B.Cu") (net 1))
 (segment (start 50.8 55.56) (end 39.182 55.56) (width 1.6) (layer "B.Cu") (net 1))
 (segment (start 30.48 56.642) (end 30.48 59.944) (width 0.5) (layer "B.Cu") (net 1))
 (segment (start 30.48 59.944) (end 31.721 61.185) (width 0.5) (layer "B.Cu") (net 1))
 (segment (start 31.721 61.185) (end 35.778331 61.185) (width 0.5) (layer "B.Cu") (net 1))
 (segment (start 39.116 55.626) (end 35.797 55.626) (width 1.6) (layer "B.Cu") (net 1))
 (segment (start 39.182 55.56) (end 39.116 55.626) (width 1.6) (layer "B.Cu") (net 1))
 (segment (start 35.778331 55.645) (end 31.477 55.645) (width 0.5) (layer "B.Cu") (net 1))
 (segment (start 31.477 55.645) (end 30.48 56.642) (width 0.5) (layer "B.Cu") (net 1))
 (segment (start 35.797 55.626) (end 35.778 55.645) (width 1.6) (layer "B.Cu") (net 1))
 (segment (start 48.114 60.56) (end 50.8 60.56) (width 1.6) (layer "F.Cu") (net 7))
 (segment (start 45.969 58.415) (end 35.778331 58.415) (width 1.6) (layer "F.Cu") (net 7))
 (segment (start 45.969 58.415) (end 48.114 60.56) (width 1.6) (layer "F.Cu") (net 7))
 (segment (start 47.86 60.56) (end 50.8 60.56) (width 1.6) (layer "B.Cu") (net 7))
 (segment (start 36.1365 58.42) (end 45.72 58.42) (width 1.6) (layer "B.Cu") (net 7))
 (segment (start 45.72 58.42) (end 47.86 60.56) (width 1.6) (layer "B.Cu") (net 7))
 (segment (start 35.778331 75.035) (end 38.205 75.035) (width 1.6) (layer "F.Cu") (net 12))
 (segment (start 38.205 75.035) (end 43.73 80.56) (width 1.6) (layer "F.Cu") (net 12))
 (segment (start 43.73 80.56) (end 50.8 80.56) (width 1.6) (layer "F.Cu") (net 12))
 (segment (start 43.73 80.56) (end 50.8 80.56) (width 1.6) (layer "B.Cu") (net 12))
 (segment (start 38.1875 75.0175) (end 43.73 80.56) (width 1.6) (layer "B.Cu") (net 12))
 (segment (start 35.86 75.0175) (end 38.1875 75.0175) (width 1.6) (layer "B.Cu") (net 12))
 (segment (start 45.466 70.612) (end 45.518 70.56) (width 1.6) (layer "F.Cu") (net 9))
 (segment (start 44.45 70.612) (end 45.466 70.612) (width 1.6) (layer "F.Cu") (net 9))
 (segment (start 40.563 66.725) (end 44.45 70.612) (width 1.6) (layer "F.Cu") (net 9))
 (segment (start 35.778331 66.725) (end 40.563 66.725) (width 1.6) (layer "F.Cu") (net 9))
 (segment (start 45.518 70.56) (end 50.8 70.56) (width 1.6) (layer "F.Cu") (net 9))
 (segment (start 40.5455 66.7075) (end 44.398 70.56) (width 1.6) (layer "B.Cu") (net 9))
 (segment (start 44.398 70.56) (end 50.8 70.56) (width 1.6) (layer "B.Cu") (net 9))
 (segment (start 35.86 66.7075) (end 40.5455 66.7075) (width 1.6) (layer "B.Cu") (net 9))
 (segment (start 44.022 40.56) (end 50.8 40.56) (width 1.6) (layer "F.Cu") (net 4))
 (segment (start 37.247 47.335) (end 44.022 40.56) (width 1.6) (layer "F.Cu") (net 4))
 (segment (start 35.778331 47.335) (end 37.247 47.335) (width 1.6) (layer "F.Cu") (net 4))
 (segment (start 44.022 40.56) (end 50.8 40.56) (width 1.6) (layer "B.Cu") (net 4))
 (segment (start 37.2645 47.3175) (end 44.022 40.56) (width 1.6) (layer "B.Cu") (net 4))
 (segment (start 35.86 47.3175) (end 37.2645 47.3175) (width 1.6) (layer "B.Cu") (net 4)))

